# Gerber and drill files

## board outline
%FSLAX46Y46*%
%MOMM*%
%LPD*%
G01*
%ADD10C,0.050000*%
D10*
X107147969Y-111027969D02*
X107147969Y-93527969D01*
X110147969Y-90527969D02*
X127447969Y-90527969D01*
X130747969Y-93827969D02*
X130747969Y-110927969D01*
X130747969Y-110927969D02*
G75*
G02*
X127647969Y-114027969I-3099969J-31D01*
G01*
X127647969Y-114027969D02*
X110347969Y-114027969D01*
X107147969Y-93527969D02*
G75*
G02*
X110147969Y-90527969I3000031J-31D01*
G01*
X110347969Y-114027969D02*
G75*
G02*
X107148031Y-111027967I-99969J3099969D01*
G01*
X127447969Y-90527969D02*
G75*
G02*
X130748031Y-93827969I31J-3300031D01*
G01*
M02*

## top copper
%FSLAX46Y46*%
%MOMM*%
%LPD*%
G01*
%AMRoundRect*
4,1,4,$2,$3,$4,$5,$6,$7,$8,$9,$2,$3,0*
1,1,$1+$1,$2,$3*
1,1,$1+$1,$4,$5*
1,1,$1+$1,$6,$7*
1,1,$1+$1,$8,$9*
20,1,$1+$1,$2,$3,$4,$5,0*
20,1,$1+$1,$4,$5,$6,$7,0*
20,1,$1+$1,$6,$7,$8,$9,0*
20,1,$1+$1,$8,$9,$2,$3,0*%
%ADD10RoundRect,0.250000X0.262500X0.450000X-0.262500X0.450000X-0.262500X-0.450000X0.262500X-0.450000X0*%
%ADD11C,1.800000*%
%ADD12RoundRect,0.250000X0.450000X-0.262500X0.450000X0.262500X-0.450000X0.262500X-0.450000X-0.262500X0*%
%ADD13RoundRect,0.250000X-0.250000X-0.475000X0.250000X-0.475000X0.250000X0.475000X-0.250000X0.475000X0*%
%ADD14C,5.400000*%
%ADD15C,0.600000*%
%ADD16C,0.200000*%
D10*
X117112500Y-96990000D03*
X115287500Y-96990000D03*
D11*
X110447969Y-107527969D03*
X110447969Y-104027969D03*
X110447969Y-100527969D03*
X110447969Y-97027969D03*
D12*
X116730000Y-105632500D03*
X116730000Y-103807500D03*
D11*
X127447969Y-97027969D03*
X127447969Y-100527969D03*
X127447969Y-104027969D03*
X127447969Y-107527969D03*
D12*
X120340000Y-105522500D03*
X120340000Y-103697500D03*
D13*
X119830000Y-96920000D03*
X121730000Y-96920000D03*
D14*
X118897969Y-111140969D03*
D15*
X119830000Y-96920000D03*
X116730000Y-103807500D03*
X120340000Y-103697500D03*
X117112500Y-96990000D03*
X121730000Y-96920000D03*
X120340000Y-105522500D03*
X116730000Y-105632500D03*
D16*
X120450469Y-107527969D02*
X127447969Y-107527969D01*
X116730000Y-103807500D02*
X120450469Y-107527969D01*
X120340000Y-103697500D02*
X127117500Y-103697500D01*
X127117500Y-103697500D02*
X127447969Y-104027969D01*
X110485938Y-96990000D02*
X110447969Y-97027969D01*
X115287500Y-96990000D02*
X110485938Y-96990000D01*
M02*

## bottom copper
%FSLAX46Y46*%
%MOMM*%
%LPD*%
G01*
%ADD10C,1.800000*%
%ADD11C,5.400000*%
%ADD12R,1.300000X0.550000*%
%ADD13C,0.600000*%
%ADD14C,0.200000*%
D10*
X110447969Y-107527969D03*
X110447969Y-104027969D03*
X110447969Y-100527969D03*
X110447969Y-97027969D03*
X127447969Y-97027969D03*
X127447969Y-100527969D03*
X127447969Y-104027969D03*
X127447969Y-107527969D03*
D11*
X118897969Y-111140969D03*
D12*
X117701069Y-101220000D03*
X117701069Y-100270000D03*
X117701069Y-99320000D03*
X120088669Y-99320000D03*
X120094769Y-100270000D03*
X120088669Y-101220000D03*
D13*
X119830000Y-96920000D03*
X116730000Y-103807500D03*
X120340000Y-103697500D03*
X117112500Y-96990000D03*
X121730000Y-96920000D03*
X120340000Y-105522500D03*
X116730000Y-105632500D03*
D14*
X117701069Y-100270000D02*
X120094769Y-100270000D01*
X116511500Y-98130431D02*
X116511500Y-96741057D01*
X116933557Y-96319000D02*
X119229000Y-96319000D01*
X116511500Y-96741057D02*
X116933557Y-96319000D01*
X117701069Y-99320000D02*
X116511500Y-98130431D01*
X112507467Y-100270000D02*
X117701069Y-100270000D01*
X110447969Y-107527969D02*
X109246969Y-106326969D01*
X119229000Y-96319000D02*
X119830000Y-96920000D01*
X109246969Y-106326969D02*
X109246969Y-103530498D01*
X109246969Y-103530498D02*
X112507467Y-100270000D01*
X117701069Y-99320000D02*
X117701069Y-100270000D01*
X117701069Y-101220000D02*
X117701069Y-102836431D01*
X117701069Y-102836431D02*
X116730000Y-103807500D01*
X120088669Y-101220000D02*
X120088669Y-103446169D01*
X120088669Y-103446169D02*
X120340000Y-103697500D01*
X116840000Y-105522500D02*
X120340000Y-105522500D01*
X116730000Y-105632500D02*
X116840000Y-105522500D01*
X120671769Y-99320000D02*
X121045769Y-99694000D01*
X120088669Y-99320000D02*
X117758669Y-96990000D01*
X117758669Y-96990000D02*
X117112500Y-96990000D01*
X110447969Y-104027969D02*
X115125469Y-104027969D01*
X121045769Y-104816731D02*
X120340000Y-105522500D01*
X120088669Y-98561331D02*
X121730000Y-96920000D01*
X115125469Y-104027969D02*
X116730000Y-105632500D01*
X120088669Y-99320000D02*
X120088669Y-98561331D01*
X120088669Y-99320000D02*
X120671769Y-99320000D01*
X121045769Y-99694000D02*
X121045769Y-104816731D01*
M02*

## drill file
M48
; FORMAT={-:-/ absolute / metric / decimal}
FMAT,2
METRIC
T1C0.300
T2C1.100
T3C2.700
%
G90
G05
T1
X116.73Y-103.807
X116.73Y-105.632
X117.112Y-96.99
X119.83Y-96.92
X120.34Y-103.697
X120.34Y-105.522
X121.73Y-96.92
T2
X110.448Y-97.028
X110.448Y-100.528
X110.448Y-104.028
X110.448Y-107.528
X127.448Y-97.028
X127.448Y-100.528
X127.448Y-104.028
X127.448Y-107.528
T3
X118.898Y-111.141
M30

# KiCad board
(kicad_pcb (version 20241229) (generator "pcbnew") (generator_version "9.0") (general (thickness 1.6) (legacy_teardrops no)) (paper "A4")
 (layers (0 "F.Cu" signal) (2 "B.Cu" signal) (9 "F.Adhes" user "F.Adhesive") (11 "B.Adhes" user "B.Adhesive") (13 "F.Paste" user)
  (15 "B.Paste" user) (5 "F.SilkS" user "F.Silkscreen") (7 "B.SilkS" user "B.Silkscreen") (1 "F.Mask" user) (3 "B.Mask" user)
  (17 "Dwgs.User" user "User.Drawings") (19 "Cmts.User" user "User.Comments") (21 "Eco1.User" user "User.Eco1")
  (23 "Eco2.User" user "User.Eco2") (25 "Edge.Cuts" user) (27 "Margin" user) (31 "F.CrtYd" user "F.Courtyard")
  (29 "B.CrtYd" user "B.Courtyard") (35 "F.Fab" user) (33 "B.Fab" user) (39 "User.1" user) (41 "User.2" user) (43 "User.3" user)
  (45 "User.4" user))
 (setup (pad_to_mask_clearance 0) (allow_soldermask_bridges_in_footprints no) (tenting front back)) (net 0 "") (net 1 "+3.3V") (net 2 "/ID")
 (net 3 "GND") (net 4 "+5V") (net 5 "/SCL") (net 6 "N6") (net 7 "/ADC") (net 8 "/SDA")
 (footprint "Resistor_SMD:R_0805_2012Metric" (layer "F.Cu") (at 116.2 96.99 180)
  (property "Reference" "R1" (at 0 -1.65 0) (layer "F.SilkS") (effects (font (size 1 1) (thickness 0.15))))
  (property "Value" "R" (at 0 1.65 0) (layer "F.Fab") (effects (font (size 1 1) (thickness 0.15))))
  (pad "1" smd roundrect (at -0.9125 0 180) (size 1.025 1.4) (layers "F.Cu" "F.Mask" "F.Paste") (roundrect_rratio 0.243902) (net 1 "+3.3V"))
  (pad "2" smd roundrect (at 0.9125 0 180) (size 1.025 1.4) (layers "F.Cu" "F.Mask" "F.Paste") (roundrect_rratio 0.243902) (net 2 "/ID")))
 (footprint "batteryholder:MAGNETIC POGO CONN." (layer "F.Cu") (at 110.447969 102.277969 90)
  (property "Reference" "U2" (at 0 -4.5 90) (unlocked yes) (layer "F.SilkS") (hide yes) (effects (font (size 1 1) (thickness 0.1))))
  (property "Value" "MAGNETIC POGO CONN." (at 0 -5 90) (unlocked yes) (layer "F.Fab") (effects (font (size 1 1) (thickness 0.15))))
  (pad "1" thru_hole circle (at -5.25 0 90) (size 1.8 1.8) (drill 1.1) (layers "*.Cu" "*.Mask") (remove_unused_layers no) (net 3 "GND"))
  (pad "2" thru_hole circle (at -1.75 0 90) (size 1.8 1.8) (drill 1.1) (layers "*.Cu" "*.Mask") (remove_unused_layers no) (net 1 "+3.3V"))
  (pad "3" thru_hole circle (at 1.75 0 90) (size 1.8 1.8) (drill 1.1) (layers "*.Cu" "*.Mask") (remove_unused_layers no) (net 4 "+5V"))
  (pad "4" thru_hole circle (at 5.25 0 90) (size 1.8 1.8) (drill 1.1) (layers "*.Cu" "*.Mask") (remove_unused_layers no) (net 2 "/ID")))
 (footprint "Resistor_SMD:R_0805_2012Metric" (layer "F.Cu") (at 116.73 104.72 90)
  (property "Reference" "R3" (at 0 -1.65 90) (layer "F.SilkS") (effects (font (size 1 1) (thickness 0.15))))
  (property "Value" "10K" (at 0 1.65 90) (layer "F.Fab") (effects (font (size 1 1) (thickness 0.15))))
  (pad "1" smd roundrect (at -0.9125 0 90) (size 1.025 1.4) (layers "F.Cu" "F.Mask" "F.Paste") (roundrect_rratio 0.243902) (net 1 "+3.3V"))
  (pad "2" smd roundrect (at 0.9125 0 90) (size 1.025 1.4) (layers "F.Cu" "F.Mask" "F.Paste") (roundrect_rratio 0.243902) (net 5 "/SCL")))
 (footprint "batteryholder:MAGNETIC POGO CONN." (layer "F.Cu") (at 127.447969 102.277969 -90)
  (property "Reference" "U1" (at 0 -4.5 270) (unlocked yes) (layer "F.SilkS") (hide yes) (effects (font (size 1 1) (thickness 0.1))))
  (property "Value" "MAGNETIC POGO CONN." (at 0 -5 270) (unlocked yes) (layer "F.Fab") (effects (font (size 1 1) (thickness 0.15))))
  (pad "1" thru_hole circle (at -5.25 0 270) (size 1.8 1.8) (drill 1.1) (layers "*.Cu" "*.Mask") (remove_unused_layers no) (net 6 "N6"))
  (pad "2" thru_hole circle (at -1.75 0 270) (size 1.8 1.8) (drill 1.1) (layers "*.Cu" "*.Mask") (remove_unused_layers no) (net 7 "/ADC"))
  (pad "3" thru_hole circle (at 1.75 0 270) (size 1.8 1.8) (drill 1.1) (layers "*.Cu" "*.Mask") (remove_unused_layers no) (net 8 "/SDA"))
  (pad "4" thru_hole circle (at 5.25 0 270) (size 1.8 1.8) (drill 1.1) (layers "*.Cu" "*.Mask") (remove_unused_layers no) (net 5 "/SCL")))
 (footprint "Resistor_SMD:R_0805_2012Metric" (layer "F.Cu") (at 120.34 104.61 90)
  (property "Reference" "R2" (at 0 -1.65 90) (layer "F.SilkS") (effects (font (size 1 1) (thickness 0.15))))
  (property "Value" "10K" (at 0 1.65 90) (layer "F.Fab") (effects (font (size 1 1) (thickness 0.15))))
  (pad "1" smd roundrect (at -0.9125 0 90) (size 1.025 1.4) (layers "F.Cu" "F.Mask" "F.Paste") (roundrect_rratio 0.243902) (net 1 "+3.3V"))
  (pad "2" smd roundrect (at 0.9125 0 90) (size 1.025 1.4) (layers "F.Cu" "F.Mask" "F.Paste") (roundrect_rratio 0.243902) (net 8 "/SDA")))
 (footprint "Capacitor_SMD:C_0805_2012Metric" (layer "F.Cu") (at 120.78 96.92)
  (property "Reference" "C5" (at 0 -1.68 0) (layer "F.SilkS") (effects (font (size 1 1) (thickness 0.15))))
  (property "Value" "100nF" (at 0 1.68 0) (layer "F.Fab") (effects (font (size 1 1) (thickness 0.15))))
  (pad "1" smd roundrect (at -0.95 0) (size 1 1.45) (layers "F.Cu" "F.Mask" "F.Paste") (roundrect_rratio 0.25) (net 3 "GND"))
  (pad "2" smd roundrect (at 0.95 0) (size 1 1.45) (layers "F.Cu" "F.Mask" "F.Paste") (roundrect_rratio 0.25) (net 1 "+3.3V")))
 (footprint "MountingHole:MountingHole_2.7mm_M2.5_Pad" (layer "F.Cu") (at 118.897969 111.140969)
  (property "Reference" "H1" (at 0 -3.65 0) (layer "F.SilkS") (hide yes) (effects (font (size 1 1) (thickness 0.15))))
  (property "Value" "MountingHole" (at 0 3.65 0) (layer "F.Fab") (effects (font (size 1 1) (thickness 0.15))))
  (pad "1" thru_hole circle (at 0 0) (size 5.4 5.4) (drill 2.7) (layers "*.Cu" "*.Mask") (remove_unused_layers no) (zone_connect 2)))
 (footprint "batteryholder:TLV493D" (layer "B.Cu") (at 118.897969 100.27 180)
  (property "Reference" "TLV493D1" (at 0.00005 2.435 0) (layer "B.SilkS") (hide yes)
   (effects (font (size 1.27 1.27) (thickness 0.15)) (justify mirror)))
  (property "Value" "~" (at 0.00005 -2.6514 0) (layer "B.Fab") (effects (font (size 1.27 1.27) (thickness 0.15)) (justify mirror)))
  (pad "1" smd rect (at 1.1969 -0.95) (size 1.3 0.55) (layers "B.Cu" "B.Mask" "B.Paste") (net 5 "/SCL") (solder_mask_margin 0.0508)
   (solder_paste_margin 0) (thermal_bridge_angle 0))
  (pad "2" smd rect (at 1.1969 0) (size 1.3 0.55) (layers "B.Cu" "B.Mask" "B.Paste") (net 3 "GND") (solder_mask_margin 0.0508)
   (solder_paste_margin 0) (thermal_bridge_angle 0))
  (pad "3" smd rect (at 1.1969 0.95) (size 1.3 0.55) (layers "B.Cu" "B.Mask" "B.Paste") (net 3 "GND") (solder_mask_margin 0.0508)
   (solder_paste_margin 0) (thermal_bridge_angle 0))
  (pad "4" smd rect (at -1.1907 0.95) (size 1.3 0.55) (layers "B.Cu" "B.Mask" "B.Paste") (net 1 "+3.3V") (solder_mask_margin 0.0508)
   (solder_paste_margin 0) (thermal_bridge_angle 0))
  (pad "5" smd rect (at -1.1968 0) (size 1.3 0.55) (layers "B.Cu" "B.Mask" "B.Paste") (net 3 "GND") (solder_mask_margin 0.0508)
   (solder_paste_margin 0) (thermal_bridge_angle 0))
  (pad "6" smd rect (at -1.1907 -0.95) (size 1.3 0.55) (layers "B.Cu" "B.Mask" "B.Paste") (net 8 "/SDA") (solder_mask_margin 0.0508)
   (solder_paste_margin 0) (thermal_bridge_angle 0))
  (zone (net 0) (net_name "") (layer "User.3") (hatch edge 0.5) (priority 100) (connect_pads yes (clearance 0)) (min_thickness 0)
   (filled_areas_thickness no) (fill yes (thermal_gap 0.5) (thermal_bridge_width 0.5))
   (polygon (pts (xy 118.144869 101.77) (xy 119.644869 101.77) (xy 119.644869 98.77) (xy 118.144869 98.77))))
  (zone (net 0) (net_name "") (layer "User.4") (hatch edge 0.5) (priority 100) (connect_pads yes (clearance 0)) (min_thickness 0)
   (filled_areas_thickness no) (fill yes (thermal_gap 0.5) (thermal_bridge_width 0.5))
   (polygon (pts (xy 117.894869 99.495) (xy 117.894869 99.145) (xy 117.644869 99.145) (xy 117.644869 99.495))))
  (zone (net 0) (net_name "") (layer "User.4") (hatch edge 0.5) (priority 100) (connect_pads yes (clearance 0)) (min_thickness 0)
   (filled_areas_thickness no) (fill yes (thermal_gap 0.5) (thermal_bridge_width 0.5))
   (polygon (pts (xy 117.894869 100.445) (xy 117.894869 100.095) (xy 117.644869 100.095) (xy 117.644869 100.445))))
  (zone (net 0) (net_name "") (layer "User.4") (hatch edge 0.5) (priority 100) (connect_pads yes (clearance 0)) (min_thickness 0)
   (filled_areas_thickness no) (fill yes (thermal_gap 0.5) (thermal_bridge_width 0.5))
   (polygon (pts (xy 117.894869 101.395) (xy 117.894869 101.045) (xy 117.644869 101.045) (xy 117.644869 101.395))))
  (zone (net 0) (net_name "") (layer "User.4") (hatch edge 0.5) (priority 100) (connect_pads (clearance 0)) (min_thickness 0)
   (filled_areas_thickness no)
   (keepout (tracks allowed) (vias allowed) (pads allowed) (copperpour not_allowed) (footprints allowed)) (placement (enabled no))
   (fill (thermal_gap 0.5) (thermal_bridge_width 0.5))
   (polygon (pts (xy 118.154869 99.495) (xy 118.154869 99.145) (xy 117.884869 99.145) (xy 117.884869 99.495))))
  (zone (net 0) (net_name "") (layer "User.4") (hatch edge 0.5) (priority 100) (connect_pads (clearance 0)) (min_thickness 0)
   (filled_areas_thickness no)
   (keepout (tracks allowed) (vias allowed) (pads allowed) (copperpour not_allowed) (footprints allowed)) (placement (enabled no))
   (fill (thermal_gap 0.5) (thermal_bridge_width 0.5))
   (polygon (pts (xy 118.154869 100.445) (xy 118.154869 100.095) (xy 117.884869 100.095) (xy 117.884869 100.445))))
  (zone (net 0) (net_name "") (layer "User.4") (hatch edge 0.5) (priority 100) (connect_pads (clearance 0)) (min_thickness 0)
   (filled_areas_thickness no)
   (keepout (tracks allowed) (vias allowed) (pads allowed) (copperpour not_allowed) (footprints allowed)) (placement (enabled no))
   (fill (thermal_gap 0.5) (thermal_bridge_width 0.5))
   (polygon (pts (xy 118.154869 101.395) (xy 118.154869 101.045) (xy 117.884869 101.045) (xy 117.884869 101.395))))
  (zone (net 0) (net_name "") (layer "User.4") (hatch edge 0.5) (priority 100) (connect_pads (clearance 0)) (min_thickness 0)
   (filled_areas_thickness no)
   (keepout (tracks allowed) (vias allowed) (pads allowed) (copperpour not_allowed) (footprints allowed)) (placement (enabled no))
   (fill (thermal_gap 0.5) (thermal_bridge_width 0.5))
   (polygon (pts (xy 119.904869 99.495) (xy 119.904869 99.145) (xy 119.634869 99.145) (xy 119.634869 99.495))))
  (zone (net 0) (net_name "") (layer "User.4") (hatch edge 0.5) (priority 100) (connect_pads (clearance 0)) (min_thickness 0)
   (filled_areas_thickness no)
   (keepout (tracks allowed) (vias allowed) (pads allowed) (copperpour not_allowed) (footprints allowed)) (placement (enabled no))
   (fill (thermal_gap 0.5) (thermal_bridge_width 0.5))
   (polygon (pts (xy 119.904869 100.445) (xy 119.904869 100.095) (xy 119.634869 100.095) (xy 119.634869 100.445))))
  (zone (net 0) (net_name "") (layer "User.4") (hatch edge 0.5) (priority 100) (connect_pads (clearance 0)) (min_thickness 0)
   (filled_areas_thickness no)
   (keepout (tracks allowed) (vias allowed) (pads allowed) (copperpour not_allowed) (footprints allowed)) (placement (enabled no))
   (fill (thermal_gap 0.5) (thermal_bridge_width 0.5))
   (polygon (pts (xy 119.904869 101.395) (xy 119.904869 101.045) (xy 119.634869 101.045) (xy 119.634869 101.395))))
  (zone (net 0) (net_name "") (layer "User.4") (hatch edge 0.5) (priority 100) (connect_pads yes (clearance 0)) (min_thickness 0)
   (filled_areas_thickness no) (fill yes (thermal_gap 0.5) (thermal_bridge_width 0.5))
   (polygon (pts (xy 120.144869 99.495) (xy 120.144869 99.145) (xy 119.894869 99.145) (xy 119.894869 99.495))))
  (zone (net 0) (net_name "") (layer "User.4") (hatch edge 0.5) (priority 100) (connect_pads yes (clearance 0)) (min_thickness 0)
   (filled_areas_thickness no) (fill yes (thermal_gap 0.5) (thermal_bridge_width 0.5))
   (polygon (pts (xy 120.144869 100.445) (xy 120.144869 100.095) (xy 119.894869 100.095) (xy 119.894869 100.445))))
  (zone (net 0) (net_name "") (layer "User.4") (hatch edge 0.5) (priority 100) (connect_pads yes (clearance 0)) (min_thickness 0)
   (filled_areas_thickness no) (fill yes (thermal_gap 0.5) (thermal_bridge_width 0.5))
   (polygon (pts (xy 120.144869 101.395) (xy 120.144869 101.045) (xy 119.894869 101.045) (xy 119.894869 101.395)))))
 (gr_line (start 107.147969 111.027969) (end 107.147969 93.527969) (stroke (width 0.05) (type default)) (layer "Edge.Cuts"))
 (gr_line (start 110.147969 90.527969) (end 127.447969 90.527969) (stroke (width 0.05) (type default)) (layer "Edge.Cuts"))
 (gr_line (start 130.747969 93.827969) (end 130.747969 110.927969) (stroke (width 0.05) (type default)) (layer "Edge.Cuts"))
 (gr_arc (start 130.747969 110.927969) (mid 129.84 113.12) (end 127.647969 114.027969) (stroke (width 0.05) (type default))
  (layer "Edge.Cuts"))
 (gr_line (start 127.647969 114.027969) (end 110.347969 114.027969) (stroke (width 0.05) (type default)) (layer "Edge.Cuts"))
 (gr_arc (start 107.147969 93.527969) (mid 108.026649 91.406649) (end 110.147969 90.527969) (stroke (width 0.05) (type default))
  (layer "Edge.Cuts"))
 (gr_arc (start 110.347969 114.027969) (mid 108.126649 113.190711) (end 107.147969 111.027969) (stroke (width 0.05) (type default))
  (layer "Edge.Cuts"))
 (gr_arc (start 127.447969 90.527969) (mid 129.781421 91.494517) (end 130.747969 93.827969) (stroke (width 0.05) (type default))
  (layer "Edge.Cuts"))
 (via blind (at 119.83 96.92) (size 0.6) (drill 0.3) (layers "F.Cu" "B.Cu") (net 3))
 (segment (start 117.701069 100.27) (end 120.094769 100.27) (width 0.2) (layer "B.Cu") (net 3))
 (segment (start 116.5115 98.130431) (end 116.5115 96.741057) (width 0.2) (layer "B.Cu") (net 3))
 (segment (start 116.933557 96.319) (end 119.229 96.319) (width 0.2) (layer "B.Cu") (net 3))
 (segment (start 116.5115 96.741057) (end 116.933557 96.319) (width 0.2) (layer "B.Cu") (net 3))
 (segment (start 117.701069 99.32) (end 116.5115 98.130431) (width 0.2) (layer "B.Cu") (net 3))
 (segment (start 112.507467 100.27) (end 117.701069 100.27) (width 0.2) (layer "B.Cu") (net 3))
 (segment (start 110.447969 107.527969) (end 109.246969 106.326969) (width 0.2) (layer "B.Cu") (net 3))
 (segment (start 119.229 96.319) (end 119.83 96.92) (width 0.2) (layer "B.Cu") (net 3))
 (segment (start 109.246969 106.326969) (end 109.246969 103.530498) (width 0.2) (layer "B.Cu") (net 3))
 (segment (start 109.246969 103.530498) (end 112.507467 100.27) (width 0.2) (layer "B.Cu") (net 3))
 (segment (start 117.701069 99.32) (end 117.701069 100.27) (width 0.2) (layer "B.Cu") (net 3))
 (segment (start 120.450469 107.527969) (end 127.447969 107.527969) (width 0.2) (layer "F.Cu") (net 5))
 (segment (start 116.73 103.8075) (end 120.450469 107.527969) (width 0.2) (layer "F.Cu") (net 5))
 (via blind (at 116.73 103.8075) (size 0.6) (drill 0.3) (layers "F.Cu" "B.Cu") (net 5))
 (segment (start 117.701069 101.22) (end 117.701069 102.836431) (width 0.2) (layer "B.Cu") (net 5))
 (segment (start 117.701069 102.836431) (end 116.73 103.8075) (width 0.2) (layer "B.Cu") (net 5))
 (segment (start 120.34 103.6975) (end 127.1175 103.6975) (width 0.2) (layer "F.Cu") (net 8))
 (segment (start 127.1175 103.6975) (end 127.447969 104.027969) (width 0.2) (layer "F.Cu") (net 8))
 (via blind (at 120.34 103.6975) (size 0.6) (drill 0.3) (layers "F.Cu" "B.Cu") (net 8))
 (segment (start 120.088669 101.22) (end 120.088669 103.446169) (width 0.2) (layer "B.Cu") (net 8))
 (segment (start 120.088669 103.446169) (end 120.34 103.6975) (width 0.2) (layer "B.Cu") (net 8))
 (via blind (at 117.1125 96.99) (size 0.6) (drill 0.3) (layers "F.Cu" "B.Cu") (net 1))
 (via blind (at 121.73 96.92) (size 0.6) (drill 0.3) (layers "F.Cu" "B.Cu") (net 1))
 (via blind (at 120.34 105.5225) (size 0.6) (drill 0.3) (layers "F.Cu" "B.Cu") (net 1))
 (via blind (at 116.73 105.6325) (size 0.6) (drill 0.3) (layers "F.Cu" "B.Cu") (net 1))
 (segment (start 116.84 105.5225) (end 120.34 105.5225) (width 0.2) (layer "B.Cu") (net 1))
 (segment (start 116.73 105.6325) (end 116.84 105.5225) (width 0.2) (layer "B.Cu") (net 1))
 (segment (start 120.671769 99.32) (end 121.045769 99.694) (width 0.2) (layer "B.Cu") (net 1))
 (segment (start 120.088669 99.32) (end 117.758669 96.99) (width 0.2) (layer "B.Cu") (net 1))
 (segment (start 117.758669 96.99) (end 117.1125 96.99) (width 0.2) (layer "B.Cu") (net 1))
 (segment (start 110.447969 104.027969) (end 115.125469 104.027969) (width 0.2) (layer "B.Cu") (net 1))
 (segment (start 121.045769 104.816731) (end 120.34 105.5225) (width 0.2) (layer "B.Cu") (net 1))
 (segment (start 120.088669 98.561331) (end 121.73 96.92) (width 0.2) (layer "B.Cu") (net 1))
 (segment (start 115.125469 104.027969) (end 116.73 105.6325) (width 0.2) (layer "B.Cu") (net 1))
 (segment (start 120.088669 99.32) (end 120.088669 98.561331) (width 0.2) (layer "B.Cu") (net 1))
 (segment (start 120.088669 99.32) (end 120.671769 99.32) (width 0.2) (layer "B.Cu") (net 1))
 (segment (start 121.045769 99.694) (end 121.045769 104.816731) (width 0.2) (layer "B.Cu") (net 1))
 (segment (start 110.485938 96.99) (end 110.447969 97.027969) (width 0.2) (layer "F.Cu") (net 2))
 (segment (start 115.2875 96.99) (end 110.485938 96.99) (width 0.2) (layer "F.Cu") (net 2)))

